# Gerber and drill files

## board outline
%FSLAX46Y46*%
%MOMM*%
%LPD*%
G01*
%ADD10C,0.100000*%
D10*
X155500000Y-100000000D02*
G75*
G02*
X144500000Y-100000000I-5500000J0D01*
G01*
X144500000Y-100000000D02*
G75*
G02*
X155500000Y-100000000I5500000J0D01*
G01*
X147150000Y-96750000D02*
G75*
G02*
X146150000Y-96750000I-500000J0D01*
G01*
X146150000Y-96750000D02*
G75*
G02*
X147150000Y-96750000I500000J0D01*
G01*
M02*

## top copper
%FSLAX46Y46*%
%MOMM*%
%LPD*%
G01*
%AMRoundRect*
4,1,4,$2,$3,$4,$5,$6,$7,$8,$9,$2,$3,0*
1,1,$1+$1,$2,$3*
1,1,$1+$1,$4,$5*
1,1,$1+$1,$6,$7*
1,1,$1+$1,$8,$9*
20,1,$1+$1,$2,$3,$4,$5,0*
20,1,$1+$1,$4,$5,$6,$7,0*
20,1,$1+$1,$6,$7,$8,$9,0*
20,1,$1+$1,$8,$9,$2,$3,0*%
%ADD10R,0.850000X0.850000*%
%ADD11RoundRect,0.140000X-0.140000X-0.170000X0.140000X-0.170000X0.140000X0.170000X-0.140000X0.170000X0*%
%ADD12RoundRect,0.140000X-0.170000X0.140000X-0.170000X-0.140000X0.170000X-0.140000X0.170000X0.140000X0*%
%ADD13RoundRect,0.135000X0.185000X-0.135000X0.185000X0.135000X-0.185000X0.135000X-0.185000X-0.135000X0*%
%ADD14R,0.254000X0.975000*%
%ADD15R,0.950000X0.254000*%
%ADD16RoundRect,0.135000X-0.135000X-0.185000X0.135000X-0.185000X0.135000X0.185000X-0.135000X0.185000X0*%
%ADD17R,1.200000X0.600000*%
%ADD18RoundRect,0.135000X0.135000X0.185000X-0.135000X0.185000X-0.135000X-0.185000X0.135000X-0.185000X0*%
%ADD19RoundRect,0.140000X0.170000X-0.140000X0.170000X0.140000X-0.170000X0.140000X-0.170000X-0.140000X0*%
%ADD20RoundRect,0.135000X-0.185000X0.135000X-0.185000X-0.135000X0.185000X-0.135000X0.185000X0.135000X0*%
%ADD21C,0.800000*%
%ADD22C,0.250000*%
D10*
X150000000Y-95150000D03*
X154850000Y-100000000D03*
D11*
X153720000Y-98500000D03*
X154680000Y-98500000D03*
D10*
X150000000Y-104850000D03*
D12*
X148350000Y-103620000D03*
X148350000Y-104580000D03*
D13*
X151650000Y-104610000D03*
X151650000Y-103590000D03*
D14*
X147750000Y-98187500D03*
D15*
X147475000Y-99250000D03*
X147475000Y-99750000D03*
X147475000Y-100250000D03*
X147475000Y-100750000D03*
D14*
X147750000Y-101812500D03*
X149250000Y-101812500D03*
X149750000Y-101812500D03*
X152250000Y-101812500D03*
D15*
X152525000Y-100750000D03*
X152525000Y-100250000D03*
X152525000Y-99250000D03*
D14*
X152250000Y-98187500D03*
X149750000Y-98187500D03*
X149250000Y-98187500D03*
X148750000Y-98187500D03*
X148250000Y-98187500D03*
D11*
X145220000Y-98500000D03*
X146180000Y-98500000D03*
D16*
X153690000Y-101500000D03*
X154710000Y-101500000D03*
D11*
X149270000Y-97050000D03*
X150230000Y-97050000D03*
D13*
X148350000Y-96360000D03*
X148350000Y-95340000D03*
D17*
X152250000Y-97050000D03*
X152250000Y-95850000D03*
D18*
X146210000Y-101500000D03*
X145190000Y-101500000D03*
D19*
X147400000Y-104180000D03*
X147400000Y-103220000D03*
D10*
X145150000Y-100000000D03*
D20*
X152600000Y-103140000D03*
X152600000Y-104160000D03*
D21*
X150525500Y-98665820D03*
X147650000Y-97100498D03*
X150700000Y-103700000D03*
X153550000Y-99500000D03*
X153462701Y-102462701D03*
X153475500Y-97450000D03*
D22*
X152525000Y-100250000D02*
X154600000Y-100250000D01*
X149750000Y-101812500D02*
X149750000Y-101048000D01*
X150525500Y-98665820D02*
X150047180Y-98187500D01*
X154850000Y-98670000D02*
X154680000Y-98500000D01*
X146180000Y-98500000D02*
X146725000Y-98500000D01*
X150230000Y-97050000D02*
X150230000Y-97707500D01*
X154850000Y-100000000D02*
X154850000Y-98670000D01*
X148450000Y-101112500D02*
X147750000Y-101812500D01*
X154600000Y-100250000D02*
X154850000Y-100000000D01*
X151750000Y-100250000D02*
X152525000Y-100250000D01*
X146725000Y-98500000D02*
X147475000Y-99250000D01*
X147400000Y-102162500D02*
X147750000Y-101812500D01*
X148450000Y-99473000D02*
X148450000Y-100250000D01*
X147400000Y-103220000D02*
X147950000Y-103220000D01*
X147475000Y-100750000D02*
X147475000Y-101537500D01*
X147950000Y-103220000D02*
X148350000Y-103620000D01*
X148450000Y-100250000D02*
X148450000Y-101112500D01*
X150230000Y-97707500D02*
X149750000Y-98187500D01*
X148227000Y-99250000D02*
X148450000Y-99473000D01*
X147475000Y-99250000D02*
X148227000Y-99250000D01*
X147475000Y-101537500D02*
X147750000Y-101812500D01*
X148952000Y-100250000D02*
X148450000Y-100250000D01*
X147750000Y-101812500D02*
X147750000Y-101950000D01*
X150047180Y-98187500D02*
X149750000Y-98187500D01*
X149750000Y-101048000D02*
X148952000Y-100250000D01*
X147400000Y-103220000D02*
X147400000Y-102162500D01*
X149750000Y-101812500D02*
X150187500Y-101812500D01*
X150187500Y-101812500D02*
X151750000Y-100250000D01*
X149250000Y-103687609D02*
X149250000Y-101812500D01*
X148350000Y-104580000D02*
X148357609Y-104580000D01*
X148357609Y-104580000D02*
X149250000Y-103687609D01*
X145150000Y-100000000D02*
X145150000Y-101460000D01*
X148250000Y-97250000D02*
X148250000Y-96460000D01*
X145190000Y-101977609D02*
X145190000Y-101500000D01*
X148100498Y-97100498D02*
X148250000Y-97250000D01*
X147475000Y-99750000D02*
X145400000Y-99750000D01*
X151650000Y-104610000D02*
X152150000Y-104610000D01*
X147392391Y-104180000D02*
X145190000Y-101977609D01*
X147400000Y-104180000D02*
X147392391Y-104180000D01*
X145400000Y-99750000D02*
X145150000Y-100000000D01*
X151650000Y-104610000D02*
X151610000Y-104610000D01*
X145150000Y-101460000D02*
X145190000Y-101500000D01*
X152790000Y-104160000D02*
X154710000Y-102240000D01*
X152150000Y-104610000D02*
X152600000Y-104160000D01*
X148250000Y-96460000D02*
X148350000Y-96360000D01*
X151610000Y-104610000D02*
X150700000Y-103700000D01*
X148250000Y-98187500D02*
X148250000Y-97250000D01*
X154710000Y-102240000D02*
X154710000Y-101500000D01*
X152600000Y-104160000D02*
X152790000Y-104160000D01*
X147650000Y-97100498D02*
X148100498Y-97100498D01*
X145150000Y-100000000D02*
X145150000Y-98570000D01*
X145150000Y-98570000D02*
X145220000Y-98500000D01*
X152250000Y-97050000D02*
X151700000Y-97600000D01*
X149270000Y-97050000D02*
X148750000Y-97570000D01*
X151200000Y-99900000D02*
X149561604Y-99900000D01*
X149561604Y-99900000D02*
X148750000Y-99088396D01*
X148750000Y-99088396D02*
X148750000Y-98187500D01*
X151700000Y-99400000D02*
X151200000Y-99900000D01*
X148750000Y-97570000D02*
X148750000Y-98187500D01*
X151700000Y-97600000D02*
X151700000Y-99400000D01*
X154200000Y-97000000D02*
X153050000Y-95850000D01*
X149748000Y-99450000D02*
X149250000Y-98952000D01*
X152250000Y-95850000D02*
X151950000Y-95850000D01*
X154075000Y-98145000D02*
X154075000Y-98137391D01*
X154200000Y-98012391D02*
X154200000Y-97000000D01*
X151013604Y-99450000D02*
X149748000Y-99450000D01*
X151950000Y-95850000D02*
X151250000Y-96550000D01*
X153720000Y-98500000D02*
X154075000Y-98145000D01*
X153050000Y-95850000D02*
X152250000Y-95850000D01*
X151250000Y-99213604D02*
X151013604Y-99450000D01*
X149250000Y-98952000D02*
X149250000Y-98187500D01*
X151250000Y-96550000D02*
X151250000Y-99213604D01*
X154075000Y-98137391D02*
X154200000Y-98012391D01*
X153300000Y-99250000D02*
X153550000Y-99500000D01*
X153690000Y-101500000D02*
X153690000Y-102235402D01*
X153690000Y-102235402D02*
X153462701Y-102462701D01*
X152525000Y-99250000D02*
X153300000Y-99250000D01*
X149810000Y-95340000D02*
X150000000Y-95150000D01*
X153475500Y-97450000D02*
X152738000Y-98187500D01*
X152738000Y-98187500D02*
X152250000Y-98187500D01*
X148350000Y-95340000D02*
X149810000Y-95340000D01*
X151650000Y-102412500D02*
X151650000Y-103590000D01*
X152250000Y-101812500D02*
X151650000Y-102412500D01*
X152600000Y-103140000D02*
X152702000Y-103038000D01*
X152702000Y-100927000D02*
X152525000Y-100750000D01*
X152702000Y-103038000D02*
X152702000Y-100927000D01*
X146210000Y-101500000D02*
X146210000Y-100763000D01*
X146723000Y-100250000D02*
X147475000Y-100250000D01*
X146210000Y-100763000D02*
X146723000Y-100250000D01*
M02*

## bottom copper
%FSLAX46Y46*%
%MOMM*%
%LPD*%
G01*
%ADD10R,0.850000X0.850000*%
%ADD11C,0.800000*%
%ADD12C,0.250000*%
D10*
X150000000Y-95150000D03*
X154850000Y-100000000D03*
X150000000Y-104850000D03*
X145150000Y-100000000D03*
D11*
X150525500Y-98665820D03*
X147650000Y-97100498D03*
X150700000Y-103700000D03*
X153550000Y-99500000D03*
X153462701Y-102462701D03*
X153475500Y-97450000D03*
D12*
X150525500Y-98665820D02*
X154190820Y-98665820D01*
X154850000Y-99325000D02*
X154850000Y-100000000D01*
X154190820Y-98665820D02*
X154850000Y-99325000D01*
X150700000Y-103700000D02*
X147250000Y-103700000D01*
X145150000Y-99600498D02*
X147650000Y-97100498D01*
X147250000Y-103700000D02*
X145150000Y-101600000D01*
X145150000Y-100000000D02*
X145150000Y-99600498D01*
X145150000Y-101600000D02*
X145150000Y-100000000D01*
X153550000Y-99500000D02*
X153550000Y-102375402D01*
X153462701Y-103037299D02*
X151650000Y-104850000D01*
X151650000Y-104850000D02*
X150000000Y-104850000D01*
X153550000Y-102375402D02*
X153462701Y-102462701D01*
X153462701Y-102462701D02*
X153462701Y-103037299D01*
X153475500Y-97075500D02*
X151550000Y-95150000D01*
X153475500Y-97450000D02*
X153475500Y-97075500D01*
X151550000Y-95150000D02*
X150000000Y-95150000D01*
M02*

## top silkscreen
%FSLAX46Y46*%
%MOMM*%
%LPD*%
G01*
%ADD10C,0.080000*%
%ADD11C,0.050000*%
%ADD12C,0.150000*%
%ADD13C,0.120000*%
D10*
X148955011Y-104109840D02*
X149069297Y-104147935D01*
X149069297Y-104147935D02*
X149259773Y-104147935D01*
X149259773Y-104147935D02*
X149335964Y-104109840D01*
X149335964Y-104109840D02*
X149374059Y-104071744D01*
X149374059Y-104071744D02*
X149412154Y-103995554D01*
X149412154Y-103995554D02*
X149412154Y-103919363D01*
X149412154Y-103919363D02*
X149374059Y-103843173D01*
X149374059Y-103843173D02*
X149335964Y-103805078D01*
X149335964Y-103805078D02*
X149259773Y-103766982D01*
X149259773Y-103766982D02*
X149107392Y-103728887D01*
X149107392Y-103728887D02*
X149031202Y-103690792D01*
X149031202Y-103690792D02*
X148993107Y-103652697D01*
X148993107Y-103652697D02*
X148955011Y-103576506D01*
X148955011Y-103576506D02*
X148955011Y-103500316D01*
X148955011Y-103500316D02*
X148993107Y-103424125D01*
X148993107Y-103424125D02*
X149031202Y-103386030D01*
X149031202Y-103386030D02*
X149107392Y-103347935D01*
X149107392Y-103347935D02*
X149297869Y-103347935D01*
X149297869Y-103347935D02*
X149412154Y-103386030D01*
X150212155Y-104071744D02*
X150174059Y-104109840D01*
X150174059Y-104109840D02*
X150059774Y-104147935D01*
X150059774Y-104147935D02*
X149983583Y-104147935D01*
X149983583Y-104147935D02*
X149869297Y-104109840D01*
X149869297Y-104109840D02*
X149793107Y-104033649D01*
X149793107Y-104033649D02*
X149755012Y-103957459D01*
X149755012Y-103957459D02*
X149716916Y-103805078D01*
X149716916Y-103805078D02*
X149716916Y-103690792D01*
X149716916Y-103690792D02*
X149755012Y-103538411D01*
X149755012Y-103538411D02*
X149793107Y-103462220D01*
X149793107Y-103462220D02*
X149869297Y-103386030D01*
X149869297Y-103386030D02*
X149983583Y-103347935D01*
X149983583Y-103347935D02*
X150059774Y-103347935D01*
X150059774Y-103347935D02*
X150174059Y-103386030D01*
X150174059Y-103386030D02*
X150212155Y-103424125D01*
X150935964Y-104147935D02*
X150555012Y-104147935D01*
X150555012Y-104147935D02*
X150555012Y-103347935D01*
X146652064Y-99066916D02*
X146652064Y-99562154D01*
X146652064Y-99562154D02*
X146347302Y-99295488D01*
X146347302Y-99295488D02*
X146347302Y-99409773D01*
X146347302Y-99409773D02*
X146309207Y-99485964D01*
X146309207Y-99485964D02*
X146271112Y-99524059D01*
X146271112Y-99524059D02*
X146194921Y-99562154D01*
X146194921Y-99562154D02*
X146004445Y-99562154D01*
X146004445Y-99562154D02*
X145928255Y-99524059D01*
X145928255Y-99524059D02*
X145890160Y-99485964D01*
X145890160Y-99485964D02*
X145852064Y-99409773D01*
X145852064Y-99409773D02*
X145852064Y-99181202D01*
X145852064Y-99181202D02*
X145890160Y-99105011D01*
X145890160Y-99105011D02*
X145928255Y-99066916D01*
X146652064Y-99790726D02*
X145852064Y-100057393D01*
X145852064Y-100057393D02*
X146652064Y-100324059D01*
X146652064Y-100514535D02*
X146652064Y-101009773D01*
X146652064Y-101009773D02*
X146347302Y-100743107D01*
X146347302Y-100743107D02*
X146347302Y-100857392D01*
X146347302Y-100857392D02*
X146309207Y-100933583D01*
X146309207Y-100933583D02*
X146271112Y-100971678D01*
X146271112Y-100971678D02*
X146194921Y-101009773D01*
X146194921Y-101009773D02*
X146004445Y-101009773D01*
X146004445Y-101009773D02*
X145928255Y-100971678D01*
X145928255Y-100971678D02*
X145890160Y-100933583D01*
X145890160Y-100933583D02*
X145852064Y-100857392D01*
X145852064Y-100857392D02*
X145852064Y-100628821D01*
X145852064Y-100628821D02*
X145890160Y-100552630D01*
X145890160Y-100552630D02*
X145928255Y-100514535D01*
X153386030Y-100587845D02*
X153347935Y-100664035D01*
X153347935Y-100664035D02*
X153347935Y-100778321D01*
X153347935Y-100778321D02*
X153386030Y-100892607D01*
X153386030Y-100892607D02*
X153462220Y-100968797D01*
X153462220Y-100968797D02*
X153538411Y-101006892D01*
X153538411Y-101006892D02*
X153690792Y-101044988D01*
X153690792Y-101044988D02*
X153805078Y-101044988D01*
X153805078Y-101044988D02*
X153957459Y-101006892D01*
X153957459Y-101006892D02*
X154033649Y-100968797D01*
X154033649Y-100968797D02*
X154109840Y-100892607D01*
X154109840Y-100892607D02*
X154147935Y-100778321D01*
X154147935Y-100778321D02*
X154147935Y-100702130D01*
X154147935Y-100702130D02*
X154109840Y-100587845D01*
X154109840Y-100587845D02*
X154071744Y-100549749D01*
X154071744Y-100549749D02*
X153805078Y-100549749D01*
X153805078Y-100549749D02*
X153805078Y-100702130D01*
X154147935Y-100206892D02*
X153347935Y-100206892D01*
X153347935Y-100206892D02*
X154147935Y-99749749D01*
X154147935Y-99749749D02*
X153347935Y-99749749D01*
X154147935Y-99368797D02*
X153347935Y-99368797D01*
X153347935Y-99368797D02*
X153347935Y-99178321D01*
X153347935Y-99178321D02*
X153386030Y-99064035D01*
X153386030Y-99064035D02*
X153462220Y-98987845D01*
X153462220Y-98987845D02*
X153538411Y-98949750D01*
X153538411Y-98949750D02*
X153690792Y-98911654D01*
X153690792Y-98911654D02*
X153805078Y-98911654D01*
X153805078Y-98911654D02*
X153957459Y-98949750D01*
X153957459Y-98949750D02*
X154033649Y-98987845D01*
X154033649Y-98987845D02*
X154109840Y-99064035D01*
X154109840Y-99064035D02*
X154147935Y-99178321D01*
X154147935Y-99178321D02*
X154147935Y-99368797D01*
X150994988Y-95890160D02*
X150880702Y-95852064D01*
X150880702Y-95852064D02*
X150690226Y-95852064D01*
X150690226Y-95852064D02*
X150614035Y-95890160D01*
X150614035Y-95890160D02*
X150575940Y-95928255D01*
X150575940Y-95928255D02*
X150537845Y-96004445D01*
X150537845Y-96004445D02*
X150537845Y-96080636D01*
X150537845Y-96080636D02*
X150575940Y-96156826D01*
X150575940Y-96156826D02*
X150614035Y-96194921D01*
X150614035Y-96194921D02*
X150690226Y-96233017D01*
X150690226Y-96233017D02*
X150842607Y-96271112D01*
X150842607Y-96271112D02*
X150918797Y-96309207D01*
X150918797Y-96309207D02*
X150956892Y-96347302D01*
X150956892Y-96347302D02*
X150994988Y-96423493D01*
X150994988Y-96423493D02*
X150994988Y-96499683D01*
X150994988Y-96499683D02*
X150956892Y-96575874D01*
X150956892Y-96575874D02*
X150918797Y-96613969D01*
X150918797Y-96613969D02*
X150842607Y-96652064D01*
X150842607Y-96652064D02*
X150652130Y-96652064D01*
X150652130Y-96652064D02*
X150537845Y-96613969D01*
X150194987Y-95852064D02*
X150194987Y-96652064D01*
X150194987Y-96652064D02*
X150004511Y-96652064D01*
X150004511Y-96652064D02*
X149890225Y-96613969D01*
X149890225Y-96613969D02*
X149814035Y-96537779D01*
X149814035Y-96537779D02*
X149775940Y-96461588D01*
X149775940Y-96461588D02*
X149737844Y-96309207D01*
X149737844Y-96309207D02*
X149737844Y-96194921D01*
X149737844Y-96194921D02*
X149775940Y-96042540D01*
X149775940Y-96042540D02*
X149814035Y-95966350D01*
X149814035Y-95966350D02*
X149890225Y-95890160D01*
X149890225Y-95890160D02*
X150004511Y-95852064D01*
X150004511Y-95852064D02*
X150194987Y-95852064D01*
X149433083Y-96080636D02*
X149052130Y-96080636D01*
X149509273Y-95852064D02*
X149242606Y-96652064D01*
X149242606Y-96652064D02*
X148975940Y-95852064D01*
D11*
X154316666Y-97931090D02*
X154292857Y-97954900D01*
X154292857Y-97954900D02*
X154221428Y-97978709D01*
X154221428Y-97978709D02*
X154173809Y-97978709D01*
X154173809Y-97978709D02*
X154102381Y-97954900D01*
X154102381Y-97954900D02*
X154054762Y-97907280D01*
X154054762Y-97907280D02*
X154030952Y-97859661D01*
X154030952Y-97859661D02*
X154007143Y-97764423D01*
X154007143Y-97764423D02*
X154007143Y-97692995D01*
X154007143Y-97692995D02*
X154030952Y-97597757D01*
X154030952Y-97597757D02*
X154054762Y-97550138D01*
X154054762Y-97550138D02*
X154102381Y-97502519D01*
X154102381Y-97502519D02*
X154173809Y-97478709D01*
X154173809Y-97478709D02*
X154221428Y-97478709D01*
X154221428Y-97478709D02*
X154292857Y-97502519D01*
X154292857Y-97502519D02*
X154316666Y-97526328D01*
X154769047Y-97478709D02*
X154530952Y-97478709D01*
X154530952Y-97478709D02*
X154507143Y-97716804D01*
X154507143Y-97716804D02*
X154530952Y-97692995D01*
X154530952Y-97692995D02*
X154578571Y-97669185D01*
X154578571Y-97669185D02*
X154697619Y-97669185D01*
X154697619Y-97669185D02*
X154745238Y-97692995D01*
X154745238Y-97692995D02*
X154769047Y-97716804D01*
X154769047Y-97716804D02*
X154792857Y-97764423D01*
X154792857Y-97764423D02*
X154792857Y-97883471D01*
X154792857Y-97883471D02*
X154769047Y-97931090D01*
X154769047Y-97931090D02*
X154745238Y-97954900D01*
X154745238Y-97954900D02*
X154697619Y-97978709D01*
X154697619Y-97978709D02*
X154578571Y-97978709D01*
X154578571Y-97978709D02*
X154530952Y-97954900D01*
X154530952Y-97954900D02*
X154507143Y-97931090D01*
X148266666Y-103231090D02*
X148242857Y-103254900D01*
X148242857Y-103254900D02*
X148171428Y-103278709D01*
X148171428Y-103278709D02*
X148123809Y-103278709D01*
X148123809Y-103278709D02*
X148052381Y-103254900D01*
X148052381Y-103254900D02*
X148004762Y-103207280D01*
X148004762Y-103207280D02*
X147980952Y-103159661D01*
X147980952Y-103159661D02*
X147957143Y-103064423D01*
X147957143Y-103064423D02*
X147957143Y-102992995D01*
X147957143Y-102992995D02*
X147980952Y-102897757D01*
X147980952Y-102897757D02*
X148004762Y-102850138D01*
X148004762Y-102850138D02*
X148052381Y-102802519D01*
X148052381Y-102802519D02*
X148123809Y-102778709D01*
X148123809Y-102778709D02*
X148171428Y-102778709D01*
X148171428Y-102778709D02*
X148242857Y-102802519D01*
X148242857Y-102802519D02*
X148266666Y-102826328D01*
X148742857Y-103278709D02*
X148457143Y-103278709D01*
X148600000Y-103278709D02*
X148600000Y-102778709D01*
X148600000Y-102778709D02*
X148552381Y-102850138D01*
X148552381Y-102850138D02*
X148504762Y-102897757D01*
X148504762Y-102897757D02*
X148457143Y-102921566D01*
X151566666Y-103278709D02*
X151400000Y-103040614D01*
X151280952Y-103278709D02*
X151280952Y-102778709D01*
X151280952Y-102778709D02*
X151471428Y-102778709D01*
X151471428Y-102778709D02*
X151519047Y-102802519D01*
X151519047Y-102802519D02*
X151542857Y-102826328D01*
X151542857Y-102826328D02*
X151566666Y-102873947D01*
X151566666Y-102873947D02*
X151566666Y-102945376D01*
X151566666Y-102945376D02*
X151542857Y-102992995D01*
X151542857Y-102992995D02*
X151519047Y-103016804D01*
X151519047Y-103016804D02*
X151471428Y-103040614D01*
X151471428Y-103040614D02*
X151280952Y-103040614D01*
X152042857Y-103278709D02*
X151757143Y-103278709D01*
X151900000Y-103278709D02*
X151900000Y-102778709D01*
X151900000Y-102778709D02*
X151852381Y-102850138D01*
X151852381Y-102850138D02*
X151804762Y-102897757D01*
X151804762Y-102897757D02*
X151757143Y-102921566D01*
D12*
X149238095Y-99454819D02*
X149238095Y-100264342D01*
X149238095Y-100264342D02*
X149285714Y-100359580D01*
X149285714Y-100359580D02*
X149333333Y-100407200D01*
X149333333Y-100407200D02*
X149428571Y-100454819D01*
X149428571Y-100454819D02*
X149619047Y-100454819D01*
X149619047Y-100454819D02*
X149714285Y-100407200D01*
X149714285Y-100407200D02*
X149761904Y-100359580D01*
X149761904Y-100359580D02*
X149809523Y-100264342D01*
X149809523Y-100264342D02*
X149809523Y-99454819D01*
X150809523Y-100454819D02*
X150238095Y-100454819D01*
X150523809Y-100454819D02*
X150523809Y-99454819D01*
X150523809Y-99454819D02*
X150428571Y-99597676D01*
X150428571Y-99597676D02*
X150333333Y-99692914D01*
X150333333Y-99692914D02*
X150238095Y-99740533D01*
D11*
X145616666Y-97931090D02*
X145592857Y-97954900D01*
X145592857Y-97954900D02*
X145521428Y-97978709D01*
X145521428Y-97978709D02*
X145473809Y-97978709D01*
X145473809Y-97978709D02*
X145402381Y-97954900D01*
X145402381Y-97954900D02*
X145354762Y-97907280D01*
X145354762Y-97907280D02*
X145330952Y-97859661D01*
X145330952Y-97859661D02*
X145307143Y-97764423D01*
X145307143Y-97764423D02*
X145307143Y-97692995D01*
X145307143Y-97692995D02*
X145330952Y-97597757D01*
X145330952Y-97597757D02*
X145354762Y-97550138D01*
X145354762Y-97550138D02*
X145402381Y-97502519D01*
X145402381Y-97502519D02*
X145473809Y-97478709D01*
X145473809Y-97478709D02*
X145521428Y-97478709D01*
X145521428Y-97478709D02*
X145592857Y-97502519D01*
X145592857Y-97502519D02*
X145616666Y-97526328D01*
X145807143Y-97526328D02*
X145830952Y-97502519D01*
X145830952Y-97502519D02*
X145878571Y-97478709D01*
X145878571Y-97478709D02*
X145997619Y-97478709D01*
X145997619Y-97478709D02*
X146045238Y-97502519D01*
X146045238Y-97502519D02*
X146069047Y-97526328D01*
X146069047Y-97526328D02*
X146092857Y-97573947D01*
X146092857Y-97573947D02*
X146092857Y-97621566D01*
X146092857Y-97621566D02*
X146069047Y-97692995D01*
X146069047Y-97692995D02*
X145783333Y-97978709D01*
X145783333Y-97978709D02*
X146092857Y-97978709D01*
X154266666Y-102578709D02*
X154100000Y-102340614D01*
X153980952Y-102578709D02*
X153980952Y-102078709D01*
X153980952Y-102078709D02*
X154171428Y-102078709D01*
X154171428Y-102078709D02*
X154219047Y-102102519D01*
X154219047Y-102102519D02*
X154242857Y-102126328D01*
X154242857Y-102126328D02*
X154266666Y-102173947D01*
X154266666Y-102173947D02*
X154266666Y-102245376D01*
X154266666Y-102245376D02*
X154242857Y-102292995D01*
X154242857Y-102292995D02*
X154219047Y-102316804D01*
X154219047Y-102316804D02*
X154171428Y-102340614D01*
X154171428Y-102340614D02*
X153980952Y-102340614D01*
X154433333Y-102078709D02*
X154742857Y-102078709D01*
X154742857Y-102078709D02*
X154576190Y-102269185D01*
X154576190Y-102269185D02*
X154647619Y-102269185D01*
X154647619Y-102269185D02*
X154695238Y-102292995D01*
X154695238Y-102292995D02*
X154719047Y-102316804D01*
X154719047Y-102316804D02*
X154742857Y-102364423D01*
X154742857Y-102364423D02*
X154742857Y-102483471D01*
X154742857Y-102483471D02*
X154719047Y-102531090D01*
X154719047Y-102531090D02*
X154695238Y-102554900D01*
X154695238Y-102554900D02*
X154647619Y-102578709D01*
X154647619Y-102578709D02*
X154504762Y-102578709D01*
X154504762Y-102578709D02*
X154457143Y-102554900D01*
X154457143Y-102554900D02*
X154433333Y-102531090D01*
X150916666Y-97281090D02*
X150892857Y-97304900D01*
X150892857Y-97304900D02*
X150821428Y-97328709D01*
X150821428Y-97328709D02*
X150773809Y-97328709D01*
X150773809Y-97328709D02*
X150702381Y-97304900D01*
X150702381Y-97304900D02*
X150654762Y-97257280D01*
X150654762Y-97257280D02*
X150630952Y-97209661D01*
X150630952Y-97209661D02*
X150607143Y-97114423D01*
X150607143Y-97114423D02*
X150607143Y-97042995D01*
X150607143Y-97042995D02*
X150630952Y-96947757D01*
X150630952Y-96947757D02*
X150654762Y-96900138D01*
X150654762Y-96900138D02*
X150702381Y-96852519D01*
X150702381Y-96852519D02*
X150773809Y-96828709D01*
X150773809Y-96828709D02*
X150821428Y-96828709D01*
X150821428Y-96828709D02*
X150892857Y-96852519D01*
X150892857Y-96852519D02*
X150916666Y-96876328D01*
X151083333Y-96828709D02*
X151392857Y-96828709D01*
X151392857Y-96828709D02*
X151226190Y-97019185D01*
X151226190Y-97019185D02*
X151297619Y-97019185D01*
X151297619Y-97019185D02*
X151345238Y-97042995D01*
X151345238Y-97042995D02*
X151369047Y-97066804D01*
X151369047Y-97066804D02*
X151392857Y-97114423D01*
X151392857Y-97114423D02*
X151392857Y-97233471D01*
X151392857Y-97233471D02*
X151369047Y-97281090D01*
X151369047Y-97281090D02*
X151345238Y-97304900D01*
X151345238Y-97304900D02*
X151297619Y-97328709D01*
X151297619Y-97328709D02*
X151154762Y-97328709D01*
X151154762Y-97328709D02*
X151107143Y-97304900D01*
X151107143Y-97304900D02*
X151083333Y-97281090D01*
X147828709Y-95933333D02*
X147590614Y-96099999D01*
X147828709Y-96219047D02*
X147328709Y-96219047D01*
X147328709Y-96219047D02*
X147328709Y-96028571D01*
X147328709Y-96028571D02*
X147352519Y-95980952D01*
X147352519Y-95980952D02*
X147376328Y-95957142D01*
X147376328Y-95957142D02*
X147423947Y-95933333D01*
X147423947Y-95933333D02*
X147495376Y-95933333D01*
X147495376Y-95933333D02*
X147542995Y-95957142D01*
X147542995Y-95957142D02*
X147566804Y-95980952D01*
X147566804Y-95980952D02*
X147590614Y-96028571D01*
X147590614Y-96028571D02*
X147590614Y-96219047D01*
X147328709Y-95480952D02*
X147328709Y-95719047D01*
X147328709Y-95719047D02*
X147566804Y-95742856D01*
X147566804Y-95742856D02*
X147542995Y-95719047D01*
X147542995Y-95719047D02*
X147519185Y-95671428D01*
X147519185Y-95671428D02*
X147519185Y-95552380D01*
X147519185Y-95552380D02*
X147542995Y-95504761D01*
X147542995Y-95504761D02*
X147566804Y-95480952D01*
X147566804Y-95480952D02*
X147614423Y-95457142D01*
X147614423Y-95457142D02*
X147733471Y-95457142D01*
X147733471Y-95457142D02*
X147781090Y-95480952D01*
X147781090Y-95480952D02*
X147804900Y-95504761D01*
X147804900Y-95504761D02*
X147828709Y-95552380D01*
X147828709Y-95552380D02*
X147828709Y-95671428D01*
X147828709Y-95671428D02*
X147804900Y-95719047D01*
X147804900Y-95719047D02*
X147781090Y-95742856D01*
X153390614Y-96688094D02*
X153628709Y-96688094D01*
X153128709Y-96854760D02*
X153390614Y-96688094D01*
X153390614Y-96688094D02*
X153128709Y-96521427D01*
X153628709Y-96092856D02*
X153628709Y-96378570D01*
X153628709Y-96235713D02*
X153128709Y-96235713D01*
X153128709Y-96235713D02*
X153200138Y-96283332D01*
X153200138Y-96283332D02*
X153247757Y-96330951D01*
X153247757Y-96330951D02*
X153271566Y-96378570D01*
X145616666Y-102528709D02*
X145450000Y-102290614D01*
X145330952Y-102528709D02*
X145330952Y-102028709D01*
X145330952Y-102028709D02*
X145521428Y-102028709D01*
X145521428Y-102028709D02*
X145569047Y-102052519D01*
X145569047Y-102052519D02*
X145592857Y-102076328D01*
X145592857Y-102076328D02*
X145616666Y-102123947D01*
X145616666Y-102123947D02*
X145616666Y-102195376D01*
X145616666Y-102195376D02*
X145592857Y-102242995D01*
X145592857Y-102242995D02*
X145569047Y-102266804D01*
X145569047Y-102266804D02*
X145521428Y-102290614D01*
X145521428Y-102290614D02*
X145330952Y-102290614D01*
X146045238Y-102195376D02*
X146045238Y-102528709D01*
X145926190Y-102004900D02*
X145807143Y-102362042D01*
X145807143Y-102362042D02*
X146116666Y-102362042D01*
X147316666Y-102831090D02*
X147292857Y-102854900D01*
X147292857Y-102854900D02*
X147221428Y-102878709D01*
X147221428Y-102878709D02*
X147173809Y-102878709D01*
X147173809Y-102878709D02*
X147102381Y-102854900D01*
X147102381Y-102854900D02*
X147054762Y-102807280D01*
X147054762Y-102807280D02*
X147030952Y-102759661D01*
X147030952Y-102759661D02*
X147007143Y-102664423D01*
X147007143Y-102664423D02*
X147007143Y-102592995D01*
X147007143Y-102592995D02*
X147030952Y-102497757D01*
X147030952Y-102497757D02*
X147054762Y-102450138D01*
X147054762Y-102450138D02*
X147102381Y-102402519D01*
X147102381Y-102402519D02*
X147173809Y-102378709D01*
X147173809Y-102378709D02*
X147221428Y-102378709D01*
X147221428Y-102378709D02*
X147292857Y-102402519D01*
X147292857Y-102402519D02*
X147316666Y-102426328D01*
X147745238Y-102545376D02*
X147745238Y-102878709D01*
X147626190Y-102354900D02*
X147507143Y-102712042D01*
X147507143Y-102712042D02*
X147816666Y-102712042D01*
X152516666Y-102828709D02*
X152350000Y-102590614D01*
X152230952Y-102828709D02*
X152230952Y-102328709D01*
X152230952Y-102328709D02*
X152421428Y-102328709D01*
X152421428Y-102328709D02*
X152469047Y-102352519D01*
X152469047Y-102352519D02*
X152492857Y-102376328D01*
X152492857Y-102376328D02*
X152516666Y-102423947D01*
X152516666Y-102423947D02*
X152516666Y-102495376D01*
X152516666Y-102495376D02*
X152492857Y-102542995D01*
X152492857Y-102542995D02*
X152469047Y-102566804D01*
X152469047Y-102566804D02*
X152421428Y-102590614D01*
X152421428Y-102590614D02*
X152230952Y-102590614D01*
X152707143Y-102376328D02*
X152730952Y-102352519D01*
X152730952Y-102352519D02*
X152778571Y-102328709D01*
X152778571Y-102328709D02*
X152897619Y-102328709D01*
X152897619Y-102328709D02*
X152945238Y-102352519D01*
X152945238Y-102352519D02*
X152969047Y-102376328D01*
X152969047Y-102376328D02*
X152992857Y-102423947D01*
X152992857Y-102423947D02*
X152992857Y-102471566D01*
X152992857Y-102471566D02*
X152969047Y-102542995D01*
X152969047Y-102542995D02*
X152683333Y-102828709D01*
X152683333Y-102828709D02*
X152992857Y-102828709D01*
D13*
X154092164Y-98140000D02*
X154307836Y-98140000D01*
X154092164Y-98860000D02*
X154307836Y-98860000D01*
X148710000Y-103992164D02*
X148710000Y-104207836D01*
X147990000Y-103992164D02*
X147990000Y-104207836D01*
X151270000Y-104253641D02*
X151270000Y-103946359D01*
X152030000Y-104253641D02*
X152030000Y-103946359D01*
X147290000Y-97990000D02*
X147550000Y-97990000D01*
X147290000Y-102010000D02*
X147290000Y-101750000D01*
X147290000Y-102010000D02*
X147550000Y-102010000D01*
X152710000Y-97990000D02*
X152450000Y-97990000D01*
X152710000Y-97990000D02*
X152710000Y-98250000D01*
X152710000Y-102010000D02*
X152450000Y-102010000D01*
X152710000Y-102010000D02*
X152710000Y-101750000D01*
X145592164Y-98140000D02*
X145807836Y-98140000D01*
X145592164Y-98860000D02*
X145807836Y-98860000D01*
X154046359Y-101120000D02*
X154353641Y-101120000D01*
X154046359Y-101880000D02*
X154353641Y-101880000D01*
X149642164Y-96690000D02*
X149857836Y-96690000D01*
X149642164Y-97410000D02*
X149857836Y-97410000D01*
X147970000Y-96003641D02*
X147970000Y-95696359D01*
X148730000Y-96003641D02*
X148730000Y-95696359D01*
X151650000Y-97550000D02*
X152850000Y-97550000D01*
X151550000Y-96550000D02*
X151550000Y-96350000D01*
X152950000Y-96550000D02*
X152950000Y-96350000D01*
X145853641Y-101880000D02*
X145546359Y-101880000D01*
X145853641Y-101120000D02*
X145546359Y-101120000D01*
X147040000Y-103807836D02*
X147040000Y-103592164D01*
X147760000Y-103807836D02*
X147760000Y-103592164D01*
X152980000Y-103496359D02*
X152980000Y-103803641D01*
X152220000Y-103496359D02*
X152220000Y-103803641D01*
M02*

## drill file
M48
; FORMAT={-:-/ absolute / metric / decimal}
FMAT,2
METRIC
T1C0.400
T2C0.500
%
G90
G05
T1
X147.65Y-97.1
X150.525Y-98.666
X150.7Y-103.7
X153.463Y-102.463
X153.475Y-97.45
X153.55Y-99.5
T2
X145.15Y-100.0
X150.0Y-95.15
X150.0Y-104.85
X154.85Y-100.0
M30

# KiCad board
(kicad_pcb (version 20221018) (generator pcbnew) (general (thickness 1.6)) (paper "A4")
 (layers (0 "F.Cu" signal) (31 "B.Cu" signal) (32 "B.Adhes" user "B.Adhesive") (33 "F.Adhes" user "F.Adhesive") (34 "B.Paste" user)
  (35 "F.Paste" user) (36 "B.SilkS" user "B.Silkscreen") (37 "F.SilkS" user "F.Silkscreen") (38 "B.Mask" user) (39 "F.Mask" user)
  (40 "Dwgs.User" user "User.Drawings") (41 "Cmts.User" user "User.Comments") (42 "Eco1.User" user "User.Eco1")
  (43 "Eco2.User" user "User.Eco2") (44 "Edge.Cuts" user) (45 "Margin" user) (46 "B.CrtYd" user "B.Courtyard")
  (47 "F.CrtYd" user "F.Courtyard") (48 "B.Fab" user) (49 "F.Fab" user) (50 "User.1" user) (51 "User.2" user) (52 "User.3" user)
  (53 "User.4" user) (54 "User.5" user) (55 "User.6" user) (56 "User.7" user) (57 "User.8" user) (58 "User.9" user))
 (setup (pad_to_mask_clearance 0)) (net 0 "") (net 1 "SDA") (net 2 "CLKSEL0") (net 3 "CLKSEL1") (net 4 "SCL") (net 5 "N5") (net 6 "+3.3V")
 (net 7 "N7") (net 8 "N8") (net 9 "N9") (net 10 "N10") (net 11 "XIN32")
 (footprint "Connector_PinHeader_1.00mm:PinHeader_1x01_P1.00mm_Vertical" (layer "F.Cu") (at 150 95.15)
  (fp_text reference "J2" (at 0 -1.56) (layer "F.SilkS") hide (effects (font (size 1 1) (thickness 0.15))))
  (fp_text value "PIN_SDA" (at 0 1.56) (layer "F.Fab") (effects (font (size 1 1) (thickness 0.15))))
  (pad "1" thru_hole rect (at 0 0) (size 0.85 0.85) (drill 0.5) (layers "*.Cu" "*.Mask") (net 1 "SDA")))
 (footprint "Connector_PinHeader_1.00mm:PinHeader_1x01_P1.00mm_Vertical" (layer "F.Cu") (at 154.85 100)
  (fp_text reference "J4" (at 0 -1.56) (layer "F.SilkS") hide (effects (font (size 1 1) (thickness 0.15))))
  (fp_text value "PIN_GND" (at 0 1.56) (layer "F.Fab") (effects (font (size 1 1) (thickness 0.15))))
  (pad "1" thru_hole rect (at 0 0) (size 0.85 0.85) (drill 0.5) (layers "*.Cu" "*.Mask") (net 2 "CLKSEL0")))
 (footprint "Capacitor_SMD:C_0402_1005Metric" (layer "F.Cu") (at 154.2 98.5)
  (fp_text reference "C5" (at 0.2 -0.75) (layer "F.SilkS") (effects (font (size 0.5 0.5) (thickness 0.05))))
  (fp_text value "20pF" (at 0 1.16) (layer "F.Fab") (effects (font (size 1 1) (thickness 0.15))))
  (fp_line (start -0.107836 -0.36) (end 0.107836 -0.36) (stroke (width 0.12) (type solid)) (layer "F.SilkS"))
  (fp_line (start -0.107836 0.36) (end 0.107836 0.36) (stroke (width 0.12) (type solid)) (layer "F.SilkS"))
  (pad "1" smd roundrect (at -0.48 0) (size 0.56 0.62) (layers "F.Cu" "F.Paste" "F.Mask") (roundrect_rratio 0.25) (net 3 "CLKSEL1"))
  (pad "2" smd roundrect (at 0.48 0) (size 0.56 0.62) (layers "F.Cu" "F.Paste" "F.Mask") (roundrect_rratio 0.25) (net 2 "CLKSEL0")))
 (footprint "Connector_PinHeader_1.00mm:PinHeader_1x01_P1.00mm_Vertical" (layer "F.Cu") (at 150 104.85)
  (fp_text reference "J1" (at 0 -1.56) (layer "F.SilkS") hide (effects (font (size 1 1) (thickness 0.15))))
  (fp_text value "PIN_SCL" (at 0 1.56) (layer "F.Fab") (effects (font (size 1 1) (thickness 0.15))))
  (pad "1" thru_hole rect (at 0 0) (size 0.85 0.85) (drill 0.5) (layers "*.Cu" "*.Mask") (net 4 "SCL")))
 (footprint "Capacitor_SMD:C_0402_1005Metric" (layer "F.Cu") (at 148.35 104.1 -90)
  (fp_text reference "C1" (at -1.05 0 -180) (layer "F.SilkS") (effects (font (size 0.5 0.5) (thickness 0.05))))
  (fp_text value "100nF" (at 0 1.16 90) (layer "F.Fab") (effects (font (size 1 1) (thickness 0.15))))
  (fp_line (start -0.107836 -0.36) (end 0.107836 -0.36) (stroke (width 0.12) (type solid)) (layer "F.SilkS"))
  (fp_line (start -0.107836 0.36) (end 0.107836 0.36) (stroke (width 0.12) (type solid)) (layer "F.SilkS"))
  (pad "1" smd roundrect (at -0.48 0 270) (size 0.56 0.62) (layers "F.Cu" "F.Paste" "F.Mask") (roundrect_rratio 0.25) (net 2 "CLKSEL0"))
  (pad "2" smd roundrect (at 0.48 0 270) (size 0.56 0.62) (layers "F.Cu" "F.Paste" "F.Mask") (roundrect_rratio 0.25) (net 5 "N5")))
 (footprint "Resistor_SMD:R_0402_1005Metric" (layer "F.Cu") (at 151.65 104.1 90)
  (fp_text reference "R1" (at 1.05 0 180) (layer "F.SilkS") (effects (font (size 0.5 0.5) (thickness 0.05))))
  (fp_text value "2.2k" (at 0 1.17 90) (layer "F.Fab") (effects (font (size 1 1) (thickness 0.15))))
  (fp_line (start -0.153641 -0.38) (end 0.153641 -0.38) (stroke (width 0.12) (type solid)) (layer "F.SilkS"))
  (fp_line (start -0.153641 0.38) (end 0.153641 0.38) (stroke (width 0.12) (type solid)) (layer "F.SilkS"))
  (pad "1" smd roundrect (at -0.51 0 90) (size 0.54 0.64) (layers "F.Cu" "F.Paste" "F.Mask") (roundrect_rratio 0.25) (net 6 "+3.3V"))
  (pad "2" smd roundrect (at 0.51 0 90) (size 0.54 0.64) (layers "F.Cu" "F.Paste" "F.Mask") (roundrect_rratio 0.25) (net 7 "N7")))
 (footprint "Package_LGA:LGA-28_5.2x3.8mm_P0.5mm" (layer "F.Cu") (at 150 100)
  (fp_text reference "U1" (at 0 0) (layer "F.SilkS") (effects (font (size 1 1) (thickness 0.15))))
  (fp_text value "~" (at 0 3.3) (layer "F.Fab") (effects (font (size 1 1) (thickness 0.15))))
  (fp_line (start -2.71 -2.01) (end -2.45 -2.01) (stroke (width 0.12) (type solid)) (layer "F.SilkS"))
  (fp_line (start -2.71 2.01) (end -2.71 1.75) (stroke (width 0.12) (type solid)) (layer "F.SilkS"))
  (fp_line (start -2.71 2.01) (end -2.45 2.01) (stroke (width 0.12) (type solid)) (layer "F.SilkS"))
  (fp_line (start 2.71 -2.01) (end 2.45 -2.01) (stroke (width 0.12) (type solid)) (layer "F.SilkS"))
  (fp_line (start 2.71 -2.01) (end 2.71 -1.75) (stroke (width 0.12) (type solid)) (layer "F.SilkS"))
  (fp_line (start 2.71 2.01) (end 2.45 2.01) (stroke (width 0.12) (type solid)) (layer "F.SilkS"))
  (fp_line (start 2.71 2.01) (end 2.71 1.75) (stroke (width 0.12) (type solid)) (layer "F.SilkS"))
  (pad "1" smd rect (at -2.25 -1.8125) (size 0.254 0.975) (layers "F.Cu" "F.Paste" "F.Mask") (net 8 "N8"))
  (pad "2" smd rect (at -2.525 -0.75 90) (size 0.254 0.95) (layers "F.Cu" "F.Paste" "F.Mask") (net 2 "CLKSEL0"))
  (pad "3" smd rect (at -2.525 -0.25 90) (size 0.254 0.95) (layers "F.Cu" "F.Paste" "F.Mask") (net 6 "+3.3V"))
  (pad "4" smd rect (at -2.525 0.25 90) (size 0.254 0.95) (layers "F.Cu" "F.Paste" "F.Mask") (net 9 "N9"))
  (pad "5" smd rect (at -2.525 0.75 90) (size 0.254 0.95) (layers "F.Cu" "F.Paste" "F.Mask") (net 2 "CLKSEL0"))
  (pad "6" smd rect (at -2.25 1.8125) (size 0.254 0.975) (layers "F.Cu" "F.Paste" "F.Mask") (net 2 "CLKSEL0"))
  (pad "9" smd rect (at -0.75 1.8125) (size 0.254 0.975) (layers "F.Cu" "F.Paste" "F.Mask") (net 5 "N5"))
  (pad "10" smd rect (at -0.25 1.8125) (size 0.254 0.975) (layers "F.Cu" "F.Paste" "F.Mask") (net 2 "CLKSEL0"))
  (pad "15" smd rect (at 2.25 1.8125) (size 0.254 0.975) (layers "F.Cu" "F.Paste" "F.Mask") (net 7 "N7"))
  (pad "16" smd rect (at 2.525 0.75 90) (size 0.254 0.95) (layers "F.Cu" "F.Paste" "F.Mask") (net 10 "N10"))
  (pad "17" smd rect (at 2.525 0.25 90) (size 0.254 0.95) (layers "F.Cu" "F.Paste" "F.Mask") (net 2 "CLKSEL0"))
  (pad "19" smd rect (at 2.525 -0.75 90) (size 0.254 0.95) (layers "F.Cu" "F.Paste" "F.Mask") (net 4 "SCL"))
  (pad "20" smd rect (at 2.25 -1.8125) (size 0.254 0.975) (layers "F.Cu" "F.Paste" "F.Mask") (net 1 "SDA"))
  (pad "25" smd rect (at -0.25 -1.8125) (size 0.254 0.975) (layers "F.Cu" "F.Paste" "F.Mask") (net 2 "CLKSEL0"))
  (pad "26" smd rect (at -0.75 -1.8125) (size 0.254 0.975) (layers "F.Cu" "F.Paste" "F.Mask") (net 3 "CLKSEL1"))
  (pad "27" smd rect (at -1.25 -1.8125) (size 0.254 0.975) (layers "F.Cu" "F.Paste" "F.Mask") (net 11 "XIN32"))
  (pad "28" smd rect (at -1.75 -1.8125) (size 0.254 0.975) (layers "F.Cu" "F.Paste" "F.Mask") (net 6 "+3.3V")))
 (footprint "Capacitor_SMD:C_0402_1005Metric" (layer "F.Cu") (at 145.7 98.5)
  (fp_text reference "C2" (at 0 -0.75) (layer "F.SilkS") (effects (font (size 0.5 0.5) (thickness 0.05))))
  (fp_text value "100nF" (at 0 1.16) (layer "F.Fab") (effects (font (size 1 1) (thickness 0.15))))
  (fp_line (start -0.107836 -0.36) (end 0.107836 -0.36) (stroke (width 0.12) (type solid)) (layer "F.SilkS"))
  (fp_line (start -0.107836 0.36) (end 0.107836 0.36) (stroke (width 0.12) (type solid)) (layer "F.SilkS"))
  (pad "1" smd roundrect (at -0.48 0) (size 0.56 0.62) (layers "F.Cu" "F.Paste" "F.Mask") (roundrect_rratio 0.25) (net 6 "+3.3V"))
  (pad "2" smd roundrect (at 0.48 0) (size 0.56 0.62) (layers "F.Cu" "F.Paste" "F.Mask") (roundrect_rratio 0.25) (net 2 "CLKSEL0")))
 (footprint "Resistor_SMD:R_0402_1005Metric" (layer "F.Cu") (at 154.2 101.5)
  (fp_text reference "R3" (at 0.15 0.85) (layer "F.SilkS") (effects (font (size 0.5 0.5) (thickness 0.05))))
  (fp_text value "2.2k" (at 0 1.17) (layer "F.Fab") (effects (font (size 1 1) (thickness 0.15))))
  (fp_line (start -0.153641 -0.38) (end 0.153641 -0.38) (stroke (width 0.12) (type solid)) (layer "F.SilkS"))
  (fp_line (start -0.153641 0.38) (end 0.153641 0.38) (stroke (width 0.12) (type solid)) (layer "F.SilkS"))
  (pad "1" smd roundrect (at -0.51 0) (size 0.54 0.64) (layers "F.Cu" "F.Paste" "F.Mask") (roundrect_rratio 0.25) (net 4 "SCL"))
  (pad "2" smd roundrect (at 0.51 0) (size 0.54 0.64) (layers "F.Cu" "F.Paste" "F.Mask") (roundrect_rratio 0.25) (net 6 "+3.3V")))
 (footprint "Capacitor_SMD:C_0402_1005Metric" (layer "F.Cu") (at 149.75 97.05)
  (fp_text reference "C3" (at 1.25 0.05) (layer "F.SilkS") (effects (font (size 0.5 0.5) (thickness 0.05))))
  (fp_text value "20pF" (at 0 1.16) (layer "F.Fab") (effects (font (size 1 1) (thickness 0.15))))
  (fp_line (start -0.107836 -0.36) (end 0.107836 -0.36) (stroke (width 0.12) (type solid)) (layer "F.SilkS"))
  (fp_line (start -0.107836 0.36) (end 0.107836 0.36) (stroke (width 0.12) (type solid)) (layer "F.SilkS"))
  (pad "1" smd roundrect (at -0.48 0) (size 0.56 0.62) (layers "F.Cu" "F.Paste" "F.Mask") (roundrect_rratio 0.25) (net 11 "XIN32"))
  (pad "2" smd roundrect (at 0.48 0) (size 0.56 0.62) (layers "F.Cu" "F.Paste" "F.Mask") (roundrect_rratio 0.25) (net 2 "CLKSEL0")))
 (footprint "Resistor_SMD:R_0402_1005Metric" (layer "F.Cu") (at 148.35 95.85 90)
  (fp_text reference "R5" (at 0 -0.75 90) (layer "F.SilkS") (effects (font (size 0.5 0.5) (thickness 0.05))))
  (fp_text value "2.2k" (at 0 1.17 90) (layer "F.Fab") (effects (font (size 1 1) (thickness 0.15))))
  (fp_line (start -0.153641 -0.38) (end 0.153641 -0.38) (stroke (width 0.12) (type solid)) (layer "F.SilkS"))
  (fp_line (start -0.153641 0.38) (end 0.153641 0.38) (stroke (width 0.12) (type solid)) (layer "F.SilkS"))
  (pad "1" smd roundrect (at -0.51 0 90) (size 0.54 0.64) (layers "F.Cu" "F.Paste" "F.Mask") (roundrect_rratio 0.25) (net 6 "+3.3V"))
  (pad "2" smd roundrect (at 0.51 0 90) (size 0.54 0.64) (layers "F.Cu" "F.Paste" "F.Mask") (roundrect_rratio 0.25) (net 1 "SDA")))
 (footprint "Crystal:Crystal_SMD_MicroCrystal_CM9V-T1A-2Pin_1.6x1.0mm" (layer "F.Cu") (at 152.25 96.45 90)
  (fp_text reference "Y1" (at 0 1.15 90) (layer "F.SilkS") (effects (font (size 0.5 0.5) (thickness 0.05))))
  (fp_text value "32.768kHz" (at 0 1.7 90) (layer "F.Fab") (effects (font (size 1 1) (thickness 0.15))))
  (fp_line (start -1.1 -0.6) (end -1.1 0.6) (stroke (width 0.12) (type solid)) (layer "F.SilkS"))
  (fp_line (start -0.1 -0.7) (end 0.1 -0.7) (stroke (width 0.12) (type solid)) (layer "F.SilkS"))
  (fp_line (start -0.1 0.7) (end 0.1 0.7) (stroke (width 0.12) (type solid)) (layer "F.SilkS"))
  (pad "1" smd rect (at -0.6 0 90) (size 0.6 1.2) (layers "F.Cu" "F.Paste" "F.Mask") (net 11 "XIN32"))
  (pad "2" smd rect (at 0.6 0 90) (size 0.6 1.2) (layers "F.Cu" "F.Paste" "F.Mask") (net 3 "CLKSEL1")))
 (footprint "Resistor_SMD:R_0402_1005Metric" (layer "F.Cu") (at 145.7 101.5 180)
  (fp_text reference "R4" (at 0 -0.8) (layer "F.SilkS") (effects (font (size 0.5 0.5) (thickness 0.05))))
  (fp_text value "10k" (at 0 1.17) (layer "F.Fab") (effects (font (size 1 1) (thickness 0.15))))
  (fp_line (start -0.153641 -0.38) (end 0.153641 -0.38) (stroke (width 0.12) (type solid)) (layer "F.SilkS"))
  (fp_line (start -0.153641 0.38) (end 0.153641 0.38) (stroke (width 0.12) (type solid)) (layer "F.SilkS"))
  (pad "1" smd roundrect (at -0.51 0 180) (size 0.54 0.64) (layers "F.Cu" "F.Paste" "F.Mask") (roundrect_rratio 0.25) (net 9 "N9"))
  (pad "2" smd roundrect (at 0.51 0 180) (size 0.54 0.64) (layers "F.Cu" "F.Paste" "F.Mask") (roundrect_rratio 0.25) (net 6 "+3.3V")))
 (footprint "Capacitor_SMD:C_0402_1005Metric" (layer "F.Cu") (at 147.4 103.7 90)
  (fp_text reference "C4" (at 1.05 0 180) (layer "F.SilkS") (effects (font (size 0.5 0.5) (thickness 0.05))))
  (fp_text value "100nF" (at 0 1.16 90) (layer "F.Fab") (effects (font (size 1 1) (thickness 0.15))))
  (fp_line (start -0.107836 -0.36) (end 0.107836 -0.36) (stroke (width 0.12) (type solid)) (layer "F.SilkS"))
  (fp_line (start -0.107836 0.36) (end 0.107836 0.36) (stroke (width 0.12) (type solid)) (layer "F.SilkS"))
  (pad "1" smd roundrect (at -0.48 0 90) (size 0.56 0.62) (layers "F.Cu" "F.Paste" "F.Mask") (roundrect_rratio 0.25) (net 6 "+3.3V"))
  (pad "2" smd roundrect (at 0.48 0 90) (size 0.56 0.62) (layers "F.Cu" "F.Paste" "F.Mask") (roundrect_rratio 0.25) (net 2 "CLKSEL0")))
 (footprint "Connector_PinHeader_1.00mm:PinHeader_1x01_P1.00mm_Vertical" (layer "F.Cu") (at 145.15 100)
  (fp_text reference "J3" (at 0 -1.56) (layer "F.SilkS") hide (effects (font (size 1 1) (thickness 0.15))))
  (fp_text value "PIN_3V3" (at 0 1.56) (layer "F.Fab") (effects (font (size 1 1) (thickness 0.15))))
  (pad "1" thru_hole rect (at 0 0) (size 0.85 0.85) (drill 0.5) (layers "*.Cu" "*.Mask") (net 6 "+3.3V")))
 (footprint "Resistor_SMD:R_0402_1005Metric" (layer "F.Cu") (at 152.6 103.65 -90)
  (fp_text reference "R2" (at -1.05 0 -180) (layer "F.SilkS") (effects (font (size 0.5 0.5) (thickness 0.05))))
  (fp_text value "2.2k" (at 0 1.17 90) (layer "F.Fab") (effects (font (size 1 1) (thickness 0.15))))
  (fp_line (start -0.153641 -0.38) (end 0.153641 -0.38) (stroke (width 0.12) (type solid)) (layer "F.SilkS"))
  (fp_line (start -0.153641 0.38) (end 0.153641 0.38) (stroke (width 0.12) (type solid)) (layer "F.SilkS"))
  (pad "1" smd roundrect (at -0.51 0 270) (size 0.54 0.64) (layers "F.Cu" "F.Paste" "F.Mask") (roundrect_rratio 0.25) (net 10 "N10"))
  (pad "2" smd roundrect (at 0.51 0 270) (size 0.54 0.64) (layers "F.Cu" "F.Paste" "F.Mask") (roundrect_rratio 0.25) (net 6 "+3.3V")))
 (gr_circle (center 150 100) (end 155.5 100) (stroke (width 0.1) (type default)) (fill none) (layer "Edge.Cuts"))
 (gr_circle (center 146.65 96.75) (end 147.15 96.75) (stroke (width 0.1) (type default)) (fill none) (layer "Edge.Cuts"))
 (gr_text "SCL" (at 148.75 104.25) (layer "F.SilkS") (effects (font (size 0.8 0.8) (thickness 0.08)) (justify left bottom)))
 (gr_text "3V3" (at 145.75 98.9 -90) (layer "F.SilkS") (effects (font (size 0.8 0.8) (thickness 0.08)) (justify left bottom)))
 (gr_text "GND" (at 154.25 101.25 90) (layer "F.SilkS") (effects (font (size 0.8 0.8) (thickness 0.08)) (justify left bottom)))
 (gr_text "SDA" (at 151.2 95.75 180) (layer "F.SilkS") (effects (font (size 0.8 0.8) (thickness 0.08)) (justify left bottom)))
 (segment (start 152.525 100.25) (end 154.6 100.25) (width 0.25) (layer "F.Cu") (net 2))
 (segment (start 149.75 101.8125) (end 149.75 101.048) (width 0.25) (layer "F.Cu") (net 2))
 (segment (start 150.5255 98.66582) (end 150.04718 98.1875) (width 0.25) (layer "F.Cu") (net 2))
 (segment (start 154.85 98.67) (end 154.68 98.5) (width 0.25) (layer "F.Cu") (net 2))
 (segment (start 146.18 98.5) (end 146.725 98.5) (width 0.25) (layer "F.Cu") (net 2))
 (segment (start 150.23 97.05) (end 150.23 97.7075) (width 0.25) (layer "F.Cu") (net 2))
 (segment (start 154.85 100) (end 154.85 98.67) (width 0.25) (layer "F.Cu") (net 2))
 (segment (start 148.45 101.1125) (end 147.75 101.8125) (width 0.25) (layer "F.Cu") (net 2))
 (segment (start 154.6 100.25) (end 154.85 100) (width 0.25) (layer "F.Cu") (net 2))
 (segment (start 151.75 100.25) (end 152.525 100.25) (width 0.25) (layer "F.Cu") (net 2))
 (segment (start 146.725 98.5) (end 147.475 99.25) (width 0.25) (layer "F.Cu") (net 2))
 (segment (start 147.4 102.1625) (end 147.75 101.8125) (width 0.25) (layer "F.Cu") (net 2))
 (segment (start 148.45 99.473) (end 148.45 100.25) (width 0.25) (layer "F.Cu") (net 2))
 (segment (start 147.4 103.22) (end 147.95 103.22) (width 0.25) (layer "F.Cu") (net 2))
 (segment (start 147.475 100.75) (end 147.475 101.5375) (width 0.25) (layer "F.Cu") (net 2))
 (segment (start 147.95 103.22) (end 148.35 103.62) (width 0.25) (layer "F.Cu") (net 2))
 (segment (start 148.45 100.25) (end 148.45 101.1125) (width 0.25) (layer "F.Cu") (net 2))
 (segment (start 150.23 97.7075) (end 149.75 98.1875) (width 0.25) (layer "F.Cu") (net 2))
 (segment (start 148.227 99.25) (end 148.45 99.473) (width 0.25) (layer "F.Cu") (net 2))
 (segment (start 147.475 99.25) (end 148.227 99.25) (width 0.25) (layer "F.Cu") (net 2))
 (segment (start 147.475 101.5375) (end 147.75 101.8125) (width 0.25) (layer "F.Cu") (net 2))
 (segment (start 148.952 100.25) (end 148.45 100.25) (width 0.25) (layer "F.Cu") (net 2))
 (segment (start 147.75 101.8125) (end 147.75 101.95) (width 0.25) (layer "F.Cu") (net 2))
 (segment (start 150.04718 98.1875) (end 149.75 98.1875) (width 0.25) (layer "F.Cu") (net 2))
 (segment (start 149.75 101.048) (end 148.952 100.25) (width 0.25) (layer "F.Cu") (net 2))
 (segment (start 147.4 103.22) (end 147.4 102.1625) (width 0.25) (layer "F.Cu") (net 2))
 (segment (start 149.75 101.8125) (end 150.1875 101.8125) (width 0.25) (layer "F.Cu") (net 2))
 (segment (start 150.1875 101.8125) (end 151.75 100.25) (width 0.25) (layer "F.Cu") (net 2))
 (via (at 150.5255 98.66582) (size 0.8) (drill 0.4) (layers "F.Cu" "B.Cu") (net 2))
 (segment (start 150.5255 98.66582) (end 154.19082 98.66582) (width 0.25) (layer "B.Cu") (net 2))
 (segment (start 154.85 99.325) (end 154.85 100) (width 0.25) (layer "B.Cu") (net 2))
 (segment (start 154.19082 98.66582) (end 154.85 99.325) (width 0.25) (layer "B.Cu") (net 2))
 (segment (start 149.25 103.687609) (end 149.25 101.8125) (width 0.25) (layer "F.Cu") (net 5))
 (segment (start 148.35 104.58) (end 148.357609 104.58) (width 0.25) (layer "F.Cu") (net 5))
 (segment (start 148.357609 104.58) (end 149.25 103.687609) (width 0.25) (layer "F.Cu") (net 5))
 (segment (start 145.15 100) (end 145.15 101.46) (width 0.25) (layer "F.Cu") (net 6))
 (segment (start 148.25 97.25) (end 148.25 96.46) (width 0.25) (layer "F.Cu") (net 6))
 (segment (start 145.19 101.977609) (end 145.19 101.5) (width 0.25) (layer "F.Cu") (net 6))
 (segment (start 148.100498 97.100498) (end 148.25 97.25) (width 0.25) (layer "F.Cu") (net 6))
 (segment (start 147.475 99.75) (end 145.4 99.75) (width 0.25) (layer "F.Cu") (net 6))
 (segment (start 151.65 104.61) (end 152.15 104.61) (width 0.25) (layer "F.Cu") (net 6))
 (segment (start 147.392391 104.18) (end 145.19 101.977609) (width 0.25) (layer "F.Cu") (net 6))
 (segment (start 147.4 104.18) (end 147.392391 104.18) (width 0.25) (layer "F.Cu") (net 6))
 (segment (start 145.4 99.75) (end 145.15 100) (width 0.25) (layer "F.Cu") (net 6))
 (segment (start 151.65 104.61) (end 151.61 104.61) (width 0.25) (layer "F.Cu") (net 6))
 (segment (start 145.15 101.46) (end 145.19 101.5) (width 0.25) (layer "F.Cu") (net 6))
 (segment (start 152.79 104.16) (end 154.71 102.24) (width 0.25) (layer "F.Cu") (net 6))
 (segment (start 152.15 104.61) (end 152.6 104.16) (width 0.25) (layer "F.Cu") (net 6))
 (segment (start 148.25 96.46) (end 148.35 96.36) (width 0.25) (layer "F.Cu") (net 6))
 (segment (start 151.61 104.61) (end 150.7 103.7) (width 0.25) (layer "F.Cu") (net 6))
 (segment (start 148.25 98.1875) (end 148.25 97.25) (width 0.25) (layer "F.Cu") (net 6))
 (segment (start 154.71 102.24) (end 154.71 101.5) (width 0.25) (layer "F.Cu") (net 6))
 (segment (start 152.6 104.16) (end 152.79 104.16) (width 0.25) (layer "F.Cu") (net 6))
 (segment (start 147.65 97.100498) (end 148.100498 97.100498) (width 0.25) (layer "F.Cu") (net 6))
 (segment (start 145.15 100) (end 145.15 98.57) (width 0.25) (layer "F.Cu") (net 6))
 (segment (start 145.15 98.57) (end 145.22 98.5) (width 0.25) (layer "F.Cu") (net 6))
 (via (at 147.65 97.100498) (size 0.8) (drill 0.4) (layers "F.Cu" "B.Cu") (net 6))
 (via (at 150.7 103.7) (size 0.8) (drill 0.4) (layers "F.Cu" "B.Cu") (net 6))
 (segment (start 150.7 103.7) (end 147.25 103.7) (width 0.25) (layer "B.Cu") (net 6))
 (segment (start 145.15 99.600498) (end 147.65 97.100498) (width 0.25) (layer "B.Cu") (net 6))
 (segment (start 147.25 103.7) (end 145.15 101.6) (width 0.25) (layer "B.Cu") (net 6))
 (segment (start 145.15 100) (end 145.15 99.600498) (width 0.25) (layer "B.Cu") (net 6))
 (segment (start 145.15 101.6) (end 145.15 100) (width 0.25) (layer "B.Cu") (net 6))
 (segment (start 152.25 97.05) (end 151.7 97.6) (width 0.25) (layer "F.Cu") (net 11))
 (segment (start 149.27 97.05) (end 148.75 97.57) (width 0.25) (layer "F.Cu") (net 11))
 (segment (start 151.2 99.9) (end 149.561604 99.9) (width 0.25) (layer "F.Cu") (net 11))
 (segment (start 149.561604 99.9) (end 148.75 99.088396) (width 0.25) (layer "F.Cu") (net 11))
 (segment (start 148.75 99.088396) (end 148.75 98.1875) (width 0.25) (layer "F.Cu") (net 11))
 (segment (start 151.7 99.4) (end 151.2 99.9) (width 0.25) (layer "F.Cu") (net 11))
 (segment (start 148.75 97.57) (end 148.75 98.1875) (width 0.25) (layer "F.Cu") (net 11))
 (segment (start 151.7 97.6) (end 151.7 99.4) (width 0.25) (layer "F.Cu") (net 11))
 (segment (start 154.2 97) (end 153.05 95.85) (width 0.25) (layer "F.Cu") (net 3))
 (segment (start 149.748 99.45) (end 149.25 98.952) (width 0.25) (layer "F.Cu") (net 3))
 (segment (start 152.25 95.85) (end 151.95 95.85) (width 0.25) (layer "F.Cu") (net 3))
 (segment (start 154.075 98.145) (end 154.075 98.137391) (width 0.25) (layer "F.Cu") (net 3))
 (segment (start 154.2 98.012391) (end 154.2 97) (width 0.25) (layer "F.Cu") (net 3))
 (segment (start 151.013604 99.45) (end 149.748 99.45) (width 0.25) (layer "F.Cu") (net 3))
 (segment (start 151.95 95.85) (end 151.25 96.55) (width 0.25) (layer "F.Cu") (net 3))
 (segment (start 153.72 98.5) (end 154.075 98.145) (width 0.25) (layer "F.Cu") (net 3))
 (segment (start 153.05 95.85) (end 152.25 95.85) (width 0.25) (layer "F.Cu") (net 3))
 (segment (start 151.25 99.213604) (end 151.013604 99.45) (width 0.25) (layer "F.Cu") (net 3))
 (segment (start 149.25 98.952) (end 149.25 98.1875) (width 0.25) (layer "F.Cu") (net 3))
 (segment (start 151.25 96.55) (end 151.25 99.213604) (width 0.25) (layer "F.Cu") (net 3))
 (segment (start 154.075 98.137391) (end 154.2 98.012391) (width 0.25) (layer "F.Cu") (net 3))
 (segment (start 153.3 99.25) (end 153.55 99.5) (width 0.25) (layer "F.Cu") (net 4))
 (segment (start 153.69 101.5) (end 153.69 102.235402) (width 0.25) (layer "F.Cu") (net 4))
 (segment (start 153.69 102.235402) (end 153.462701 102.462701) (width 0.25) (layer "F.Cu") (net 4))
 (segment (start 152.525 99.25) (end 153.3 99.25) (width 0.25) (layer "F.Cu") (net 4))
 (via (at 153.55 99.5) (size 0.8) (drill 0.4) (layers "F.Cu" "B.Cu") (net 4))
 (via (at 153.462701 102.462701) (size 0.8) (drill 0.4) (layers "F.Cu" "B.Cu") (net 4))
 (segment (start 153.55 99.5) (end 153.55 102.375402) (width 0.25) (layer "B.Cu") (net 4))
 (segment (start 153.462701 103.037299) (end 151.65 104.85) (width 0.25) (layer "B.Cu") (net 4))
 (segment (start 151.65 104.85) (end 150 104.85) (width 0.25) (layer "B.Cu") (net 4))
 (segment (start 153.55 102.375402) (end 153.462701 102.462701) (width 0.25) (layer "B.Cu") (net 4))
 (segment (start 153.462701 102.462701) (end 153.462701 103.037299) (width 0.25) (layer "B.Cu") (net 4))
 (segment (start 149.81 95.34) (end 150 95.15) (width 0.25) (layer "F.Cu") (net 1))
 (segment (start 153.4755 97.45) (end 152.738 98.1875) (width 0.25) (layer "F.Cu") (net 1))
 (segment (start 152.738 98.1875) (end 152.25 98.1875) (width 0.25) (layer "F.Cu") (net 1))
 (segment (start 148.35 95.34) (end 149.81 95.34) (width 0.25) (layer "F.Cu") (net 1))
 (via (at 153.4755 97.45) (size 0.8) (drill 0.4) (layers "F.Cu" "B.Cu") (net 1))
 (segment (start 153.4755 97.0755) (end 151.55 95.15) (width 0.25) (layer "B.Cu") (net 1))
 (segment (start 153.4755 97.45) (end 153.4755 97.0755) (width 0.25) (layer "B.Cu") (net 1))
 (segment (start 151.55 95.15) (end 150 95.15) (width 0.25) (layer "B.Cu") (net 1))
 (segment (start 151.65 102.4125) (end 151.65 103.59) (width 0.25) (layer "F.Cu") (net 7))
 (segment (start 152.25 101.8125) (end 151.65 102.4125) (width 0.25) (layer "F.Cu") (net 7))
 (segment (start 152.6 103.14) (end 152.702 103.038) (width 0.25) (layer "F.Cu") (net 10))
 (segment (start 152.702 100.927) (end 152.525 100.75) (width 0.25) (layer "F.Cu") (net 10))
 (segment (start 152.702 103.038) (end 152.702 100.927) (width 0.25) (layer "F.Cu") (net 10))
 (segment (start 146.21 101.5) (end 146.21 100.763) (width 0.25) (layer "F.Cu") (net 9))
 (segment (start 146.723 100.25) (end 147.475 100.25) (width 0.25) (layer "F.Cu") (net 9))
 (segment (start 146.21 100.763) (end 146.723 100.25) (width 0.25) (layer "F.Cu") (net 9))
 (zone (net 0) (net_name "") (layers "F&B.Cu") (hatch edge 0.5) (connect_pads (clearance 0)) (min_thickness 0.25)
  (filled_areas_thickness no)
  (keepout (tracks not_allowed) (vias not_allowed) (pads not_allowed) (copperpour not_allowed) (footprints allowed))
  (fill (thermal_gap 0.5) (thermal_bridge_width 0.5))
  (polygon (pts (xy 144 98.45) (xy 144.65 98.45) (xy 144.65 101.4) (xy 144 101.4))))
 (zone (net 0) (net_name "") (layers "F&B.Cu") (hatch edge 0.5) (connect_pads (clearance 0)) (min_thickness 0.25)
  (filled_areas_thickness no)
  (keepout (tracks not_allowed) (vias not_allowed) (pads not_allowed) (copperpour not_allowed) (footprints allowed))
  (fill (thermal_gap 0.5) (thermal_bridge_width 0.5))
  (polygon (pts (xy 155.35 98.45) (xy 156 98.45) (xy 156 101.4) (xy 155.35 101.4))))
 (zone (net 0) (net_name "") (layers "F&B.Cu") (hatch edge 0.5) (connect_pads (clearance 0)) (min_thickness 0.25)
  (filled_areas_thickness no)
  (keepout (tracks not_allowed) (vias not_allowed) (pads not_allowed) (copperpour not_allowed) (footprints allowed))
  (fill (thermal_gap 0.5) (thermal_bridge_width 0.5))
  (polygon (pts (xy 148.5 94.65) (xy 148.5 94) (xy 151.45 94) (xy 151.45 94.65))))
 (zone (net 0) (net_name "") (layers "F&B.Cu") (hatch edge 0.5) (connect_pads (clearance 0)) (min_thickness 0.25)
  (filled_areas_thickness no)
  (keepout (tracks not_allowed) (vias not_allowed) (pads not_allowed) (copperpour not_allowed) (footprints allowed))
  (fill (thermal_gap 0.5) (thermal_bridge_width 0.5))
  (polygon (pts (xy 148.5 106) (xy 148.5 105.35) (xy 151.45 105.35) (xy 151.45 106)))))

